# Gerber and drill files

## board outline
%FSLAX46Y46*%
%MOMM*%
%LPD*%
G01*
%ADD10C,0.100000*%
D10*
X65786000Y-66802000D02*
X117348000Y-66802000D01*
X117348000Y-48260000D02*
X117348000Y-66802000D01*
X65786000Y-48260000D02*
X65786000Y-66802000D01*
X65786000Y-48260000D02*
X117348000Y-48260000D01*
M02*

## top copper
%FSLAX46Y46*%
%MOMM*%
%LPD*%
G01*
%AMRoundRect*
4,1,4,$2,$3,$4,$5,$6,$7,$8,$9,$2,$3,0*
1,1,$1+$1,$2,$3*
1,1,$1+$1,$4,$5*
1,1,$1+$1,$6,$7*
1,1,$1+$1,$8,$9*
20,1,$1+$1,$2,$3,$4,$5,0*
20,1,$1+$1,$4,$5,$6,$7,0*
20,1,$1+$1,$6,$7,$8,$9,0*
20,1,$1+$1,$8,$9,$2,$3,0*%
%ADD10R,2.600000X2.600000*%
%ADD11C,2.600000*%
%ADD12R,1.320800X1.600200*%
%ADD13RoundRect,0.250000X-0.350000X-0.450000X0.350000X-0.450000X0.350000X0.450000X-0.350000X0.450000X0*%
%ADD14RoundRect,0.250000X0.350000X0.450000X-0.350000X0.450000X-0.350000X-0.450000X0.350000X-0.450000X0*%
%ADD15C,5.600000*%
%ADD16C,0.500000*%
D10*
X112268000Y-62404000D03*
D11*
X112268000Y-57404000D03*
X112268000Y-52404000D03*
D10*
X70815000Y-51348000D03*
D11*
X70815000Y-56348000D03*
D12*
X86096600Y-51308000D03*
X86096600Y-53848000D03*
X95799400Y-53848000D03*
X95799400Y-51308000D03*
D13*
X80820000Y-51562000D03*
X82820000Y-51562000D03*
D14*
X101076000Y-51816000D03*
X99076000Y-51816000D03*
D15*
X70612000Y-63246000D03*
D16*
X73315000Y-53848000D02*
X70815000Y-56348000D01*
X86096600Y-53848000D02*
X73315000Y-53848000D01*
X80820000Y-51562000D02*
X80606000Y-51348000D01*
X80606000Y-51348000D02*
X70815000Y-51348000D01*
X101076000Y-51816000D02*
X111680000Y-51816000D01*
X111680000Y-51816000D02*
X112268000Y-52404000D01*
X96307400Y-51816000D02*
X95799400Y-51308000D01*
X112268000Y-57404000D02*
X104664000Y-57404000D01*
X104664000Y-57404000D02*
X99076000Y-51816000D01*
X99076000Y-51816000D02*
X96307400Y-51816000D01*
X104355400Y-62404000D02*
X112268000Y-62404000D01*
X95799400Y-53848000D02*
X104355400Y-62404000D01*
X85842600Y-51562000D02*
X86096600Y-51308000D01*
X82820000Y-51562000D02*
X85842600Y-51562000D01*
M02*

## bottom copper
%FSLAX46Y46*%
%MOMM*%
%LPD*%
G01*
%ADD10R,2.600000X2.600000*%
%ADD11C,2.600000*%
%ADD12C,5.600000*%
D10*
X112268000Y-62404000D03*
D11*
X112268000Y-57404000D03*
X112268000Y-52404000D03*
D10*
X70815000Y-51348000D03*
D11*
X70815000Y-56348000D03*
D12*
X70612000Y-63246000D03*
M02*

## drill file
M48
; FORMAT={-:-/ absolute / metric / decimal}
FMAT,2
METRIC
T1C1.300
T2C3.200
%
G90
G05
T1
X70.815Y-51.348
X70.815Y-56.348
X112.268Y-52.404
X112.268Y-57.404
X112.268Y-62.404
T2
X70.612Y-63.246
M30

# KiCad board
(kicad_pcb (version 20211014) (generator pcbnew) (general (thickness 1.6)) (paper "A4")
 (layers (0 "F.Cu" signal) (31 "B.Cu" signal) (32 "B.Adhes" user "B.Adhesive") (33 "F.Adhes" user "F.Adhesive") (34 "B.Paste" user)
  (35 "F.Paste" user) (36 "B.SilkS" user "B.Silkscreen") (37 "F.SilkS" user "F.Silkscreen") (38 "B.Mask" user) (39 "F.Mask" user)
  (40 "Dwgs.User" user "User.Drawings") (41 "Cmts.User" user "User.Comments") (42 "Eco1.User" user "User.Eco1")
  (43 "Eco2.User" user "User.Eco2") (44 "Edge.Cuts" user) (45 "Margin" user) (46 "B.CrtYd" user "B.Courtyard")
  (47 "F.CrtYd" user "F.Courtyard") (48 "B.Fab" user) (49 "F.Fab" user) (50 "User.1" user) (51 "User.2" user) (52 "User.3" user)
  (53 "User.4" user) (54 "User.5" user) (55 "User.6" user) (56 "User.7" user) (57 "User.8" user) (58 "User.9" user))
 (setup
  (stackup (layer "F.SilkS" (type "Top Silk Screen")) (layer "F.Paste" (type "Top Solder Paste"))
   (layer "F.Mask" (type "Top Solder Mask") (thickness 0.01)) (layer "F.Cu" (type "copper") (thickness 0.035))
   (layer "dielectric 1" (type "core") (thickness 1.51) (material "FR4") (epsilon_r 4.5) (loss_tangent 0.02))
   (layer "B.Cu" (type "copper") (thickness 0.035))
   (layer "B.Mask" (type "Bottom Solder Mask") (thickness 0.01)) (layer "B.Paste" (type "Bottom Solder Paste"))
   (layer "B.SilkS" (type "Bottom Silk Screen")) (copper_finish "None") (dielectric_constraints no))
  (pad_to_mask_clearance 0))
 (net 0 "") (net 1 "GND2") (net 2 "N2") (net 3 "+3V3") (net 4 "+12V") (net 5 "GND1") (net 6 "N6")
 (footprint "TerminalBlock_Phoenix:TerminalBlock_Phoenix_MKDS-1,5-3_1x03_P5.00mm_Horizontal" (layer "F.Cu") (at 112.268 62.404 90)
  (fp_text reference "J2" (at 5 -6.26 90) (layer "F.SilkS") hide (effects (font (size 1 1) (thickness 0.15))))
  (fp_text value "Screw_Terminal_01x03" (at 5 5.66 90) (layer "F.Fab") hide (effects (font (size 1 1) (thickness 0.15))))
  (pad "1" thru_hole rect (at 0 0 90) (size 2.6 2.6) (drill 1.3) (layers *.Cu *.Mask) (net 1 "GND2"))
  (pad "2" thru_hole circle (at 5 0 90) (size 2.6 2.6) (drill 1.3) (layers *.Cu *.Mask) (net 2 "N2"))
  (pad "3" thru_hole circle (at 10 0 90) (size 2.6 2.6) (drill 1.3) (layers *.Cu *.Mask) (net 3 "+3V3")))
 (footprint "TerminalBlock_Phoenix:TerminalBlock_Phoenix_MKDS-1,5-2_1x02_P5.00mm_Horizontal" (layer "F.Cu") (at 70.815 51.348 -90)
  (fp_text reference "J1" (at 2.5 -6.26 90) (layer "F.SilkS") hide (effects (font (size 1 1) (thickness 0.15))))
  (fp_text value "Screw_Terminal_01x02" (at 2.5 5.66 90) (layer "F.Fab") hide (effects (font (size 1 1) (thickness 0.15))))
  (pad "1" thru_hole rect (at 0 0 270) (size 2.6 2.6) (drill 1.3) (layers *.Cu *.Mask) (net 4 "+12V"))
  (pad "2" thru_hole circle (at 5 0 270) (size 2.6 2.6) (drill 1.3) (layers *.Cu *.Mask) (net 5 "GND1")))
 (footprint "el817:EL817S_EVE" (layer "F.Cu") (at 90.948 52.578)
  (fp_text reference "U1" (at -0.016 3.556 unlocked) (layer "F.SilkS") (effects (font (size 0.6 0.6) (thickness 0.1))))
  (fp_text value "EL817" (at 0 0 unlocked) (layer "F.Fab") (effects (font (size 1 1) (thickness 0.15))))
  (pad "1" smd rect (at -4.8514 -1.27) (size 1.3208 1.6002) (layers "F.Cu" "F.Paste" "F.Mask") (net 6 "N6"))
  (pad "2" smd rect (at -4.8514 1.27) (size 1.3208 1.6002) (layers "F.Cu" "F.Paste" "F.Mask") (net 5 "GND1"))
  (pad "3" smd rect (at 4.8514 1.27) (size 1.3208 1.6002) (layers "F.Cu" "F.Paste" "F.Mask") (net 1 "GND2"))
  (pad "4" smd rect (at 4.8514 -1.27) (size 1.3208 1.6002) (layers "F.Cu" "F.Paste" "F.Mask") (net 2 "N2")))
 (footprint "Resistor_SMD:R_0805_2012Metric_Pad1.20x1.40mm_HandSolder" (layer "F.Cu") (at 81.82 51.562)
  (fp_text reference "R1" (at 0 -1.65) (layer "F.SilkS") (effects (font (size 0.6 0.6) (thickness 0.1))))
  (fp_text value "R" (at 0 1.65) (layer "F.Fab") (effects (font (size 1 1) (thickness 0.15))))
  (pad "1" smd roundrect (at -1 0) (size 1.2 1.4) (layers "F.Cu" "F.Paste" "F.Mask") (roundrect_rratio 0.2083333333) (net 4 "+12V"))
  (pad "2" smd roundrect (at 1 0) (size 1.2 1.4) (layers "F.Cu" "F.Paste" "F.Mask") (roundrect_rratio 0.2083333333) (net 6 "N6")))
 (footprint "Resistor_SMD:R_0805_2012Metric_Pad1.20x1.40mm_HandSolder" (layer "F.Cu") (at 100.076 51.816 180)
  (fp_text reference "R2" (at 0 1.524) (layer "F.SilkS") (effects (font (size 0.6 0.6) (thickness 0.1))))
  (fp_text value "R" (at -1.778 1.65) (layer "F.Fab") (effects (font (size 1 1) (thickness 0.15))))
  (pad "1" smd roundrect (at -1 0 180) (size 1.2 1.4) (layers "F.Cu" "F.Paste" "F.Mask") (roundrect_rratio 0.2083333333) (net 3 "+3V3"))
  (pad "2" smd roundrect (at 1 0 180) (size 1.2 1.4) (layers "F.Cu" "F.Paste" "F.Mask") (roundrect_rratio 0.2083333333) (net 2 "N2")))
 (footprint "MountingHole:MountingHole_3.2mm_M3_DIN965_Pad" (layer "F.Cu") (at 70.612 63.246)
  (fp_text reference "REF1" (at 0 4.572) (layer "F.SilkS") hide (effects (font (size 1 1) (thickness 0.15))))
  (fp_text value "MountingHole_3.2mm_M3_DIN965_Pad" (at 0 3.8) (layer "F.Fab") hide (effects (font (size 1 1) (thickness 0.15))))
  (pad "1" thru_hole circle (at 0 0) (size 5.6 5.6) (drill 3.2) (layers *.Cu *.Mask)))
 (gr_line (start 65.786 66.802) (end 117.348 66.802) (layer "Edge.Cuts") (width 0.1))
 (gr_line (start 117.348 48.26) (end 117.348 66.802) (layer "Edge.Cuts") (width 0.1))
 (gr_line (start 65.786 48.26) (end 65.786 66.802) (layer "Edge.Cuts") (width 0.1))
 (gr_line (start 65.786 48.26) (end 117.348 48.26) (layer "Edge.Cuts") (width 0.1))
 (segment (start 73.315 53.848) (end 70.815 56.348) (width 0.5) (layer "F.Cu") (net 5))
 (segment (start 86.0966 53.848) (end 73.315 53.848) (width 0.5) (layer "F.Cu") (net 5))
 (segment (start 80.82 51.562) (end 80.606 51.348) (width 0.5) (layer "F.Cu") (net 4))
 (segment (start 80.606 51.348) (end 70.815 51.348) (width 0.5) (layer "F.Cu") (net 4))
 (segment (start 101.076 51.816) (end 111.68 51.816) (width 0.5) (layer "F.Cu") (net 3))
 (segment (start 111.68 51.816) (end 112.268 52.404) (width 0.5) (layer "F.Cu") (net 3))
 (segment (start 96.3074 51.816) (end 95.7994 51.308) (width 0.5) (layer "F.Cu") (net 2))
 (segment (start 112.268 57.404) (end 104.664 57.404) (width 0.5) (layer "F.Cu") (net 2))
 (segment (start 104.664 57.404) (end 99.076 51.816) (width 0.5) (layer "F.Cu") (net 2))
 (segment (start 99.076 51.816) (end 96.3074 51.816) (width 0.5) (layer "F.Cu") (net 2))
 (segment (start 104.3554 62.404) (end 112.268 62.404) (width 0.5) (layer "F.Cu") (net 1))
 (segment (start 95.7994 53.848) (end 104.3554 62.404) (width 0.5) (layer "F.Cu") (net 1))
 (segment (start 85.8426 51.562) (end 86.0966 51.308) (width 0.5) (layer "F.Cu") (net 6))
 (segment (start 82.82 51.562) (end 85.8426 51.562) (width 0.5) (layer "F.Cu") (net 6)))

